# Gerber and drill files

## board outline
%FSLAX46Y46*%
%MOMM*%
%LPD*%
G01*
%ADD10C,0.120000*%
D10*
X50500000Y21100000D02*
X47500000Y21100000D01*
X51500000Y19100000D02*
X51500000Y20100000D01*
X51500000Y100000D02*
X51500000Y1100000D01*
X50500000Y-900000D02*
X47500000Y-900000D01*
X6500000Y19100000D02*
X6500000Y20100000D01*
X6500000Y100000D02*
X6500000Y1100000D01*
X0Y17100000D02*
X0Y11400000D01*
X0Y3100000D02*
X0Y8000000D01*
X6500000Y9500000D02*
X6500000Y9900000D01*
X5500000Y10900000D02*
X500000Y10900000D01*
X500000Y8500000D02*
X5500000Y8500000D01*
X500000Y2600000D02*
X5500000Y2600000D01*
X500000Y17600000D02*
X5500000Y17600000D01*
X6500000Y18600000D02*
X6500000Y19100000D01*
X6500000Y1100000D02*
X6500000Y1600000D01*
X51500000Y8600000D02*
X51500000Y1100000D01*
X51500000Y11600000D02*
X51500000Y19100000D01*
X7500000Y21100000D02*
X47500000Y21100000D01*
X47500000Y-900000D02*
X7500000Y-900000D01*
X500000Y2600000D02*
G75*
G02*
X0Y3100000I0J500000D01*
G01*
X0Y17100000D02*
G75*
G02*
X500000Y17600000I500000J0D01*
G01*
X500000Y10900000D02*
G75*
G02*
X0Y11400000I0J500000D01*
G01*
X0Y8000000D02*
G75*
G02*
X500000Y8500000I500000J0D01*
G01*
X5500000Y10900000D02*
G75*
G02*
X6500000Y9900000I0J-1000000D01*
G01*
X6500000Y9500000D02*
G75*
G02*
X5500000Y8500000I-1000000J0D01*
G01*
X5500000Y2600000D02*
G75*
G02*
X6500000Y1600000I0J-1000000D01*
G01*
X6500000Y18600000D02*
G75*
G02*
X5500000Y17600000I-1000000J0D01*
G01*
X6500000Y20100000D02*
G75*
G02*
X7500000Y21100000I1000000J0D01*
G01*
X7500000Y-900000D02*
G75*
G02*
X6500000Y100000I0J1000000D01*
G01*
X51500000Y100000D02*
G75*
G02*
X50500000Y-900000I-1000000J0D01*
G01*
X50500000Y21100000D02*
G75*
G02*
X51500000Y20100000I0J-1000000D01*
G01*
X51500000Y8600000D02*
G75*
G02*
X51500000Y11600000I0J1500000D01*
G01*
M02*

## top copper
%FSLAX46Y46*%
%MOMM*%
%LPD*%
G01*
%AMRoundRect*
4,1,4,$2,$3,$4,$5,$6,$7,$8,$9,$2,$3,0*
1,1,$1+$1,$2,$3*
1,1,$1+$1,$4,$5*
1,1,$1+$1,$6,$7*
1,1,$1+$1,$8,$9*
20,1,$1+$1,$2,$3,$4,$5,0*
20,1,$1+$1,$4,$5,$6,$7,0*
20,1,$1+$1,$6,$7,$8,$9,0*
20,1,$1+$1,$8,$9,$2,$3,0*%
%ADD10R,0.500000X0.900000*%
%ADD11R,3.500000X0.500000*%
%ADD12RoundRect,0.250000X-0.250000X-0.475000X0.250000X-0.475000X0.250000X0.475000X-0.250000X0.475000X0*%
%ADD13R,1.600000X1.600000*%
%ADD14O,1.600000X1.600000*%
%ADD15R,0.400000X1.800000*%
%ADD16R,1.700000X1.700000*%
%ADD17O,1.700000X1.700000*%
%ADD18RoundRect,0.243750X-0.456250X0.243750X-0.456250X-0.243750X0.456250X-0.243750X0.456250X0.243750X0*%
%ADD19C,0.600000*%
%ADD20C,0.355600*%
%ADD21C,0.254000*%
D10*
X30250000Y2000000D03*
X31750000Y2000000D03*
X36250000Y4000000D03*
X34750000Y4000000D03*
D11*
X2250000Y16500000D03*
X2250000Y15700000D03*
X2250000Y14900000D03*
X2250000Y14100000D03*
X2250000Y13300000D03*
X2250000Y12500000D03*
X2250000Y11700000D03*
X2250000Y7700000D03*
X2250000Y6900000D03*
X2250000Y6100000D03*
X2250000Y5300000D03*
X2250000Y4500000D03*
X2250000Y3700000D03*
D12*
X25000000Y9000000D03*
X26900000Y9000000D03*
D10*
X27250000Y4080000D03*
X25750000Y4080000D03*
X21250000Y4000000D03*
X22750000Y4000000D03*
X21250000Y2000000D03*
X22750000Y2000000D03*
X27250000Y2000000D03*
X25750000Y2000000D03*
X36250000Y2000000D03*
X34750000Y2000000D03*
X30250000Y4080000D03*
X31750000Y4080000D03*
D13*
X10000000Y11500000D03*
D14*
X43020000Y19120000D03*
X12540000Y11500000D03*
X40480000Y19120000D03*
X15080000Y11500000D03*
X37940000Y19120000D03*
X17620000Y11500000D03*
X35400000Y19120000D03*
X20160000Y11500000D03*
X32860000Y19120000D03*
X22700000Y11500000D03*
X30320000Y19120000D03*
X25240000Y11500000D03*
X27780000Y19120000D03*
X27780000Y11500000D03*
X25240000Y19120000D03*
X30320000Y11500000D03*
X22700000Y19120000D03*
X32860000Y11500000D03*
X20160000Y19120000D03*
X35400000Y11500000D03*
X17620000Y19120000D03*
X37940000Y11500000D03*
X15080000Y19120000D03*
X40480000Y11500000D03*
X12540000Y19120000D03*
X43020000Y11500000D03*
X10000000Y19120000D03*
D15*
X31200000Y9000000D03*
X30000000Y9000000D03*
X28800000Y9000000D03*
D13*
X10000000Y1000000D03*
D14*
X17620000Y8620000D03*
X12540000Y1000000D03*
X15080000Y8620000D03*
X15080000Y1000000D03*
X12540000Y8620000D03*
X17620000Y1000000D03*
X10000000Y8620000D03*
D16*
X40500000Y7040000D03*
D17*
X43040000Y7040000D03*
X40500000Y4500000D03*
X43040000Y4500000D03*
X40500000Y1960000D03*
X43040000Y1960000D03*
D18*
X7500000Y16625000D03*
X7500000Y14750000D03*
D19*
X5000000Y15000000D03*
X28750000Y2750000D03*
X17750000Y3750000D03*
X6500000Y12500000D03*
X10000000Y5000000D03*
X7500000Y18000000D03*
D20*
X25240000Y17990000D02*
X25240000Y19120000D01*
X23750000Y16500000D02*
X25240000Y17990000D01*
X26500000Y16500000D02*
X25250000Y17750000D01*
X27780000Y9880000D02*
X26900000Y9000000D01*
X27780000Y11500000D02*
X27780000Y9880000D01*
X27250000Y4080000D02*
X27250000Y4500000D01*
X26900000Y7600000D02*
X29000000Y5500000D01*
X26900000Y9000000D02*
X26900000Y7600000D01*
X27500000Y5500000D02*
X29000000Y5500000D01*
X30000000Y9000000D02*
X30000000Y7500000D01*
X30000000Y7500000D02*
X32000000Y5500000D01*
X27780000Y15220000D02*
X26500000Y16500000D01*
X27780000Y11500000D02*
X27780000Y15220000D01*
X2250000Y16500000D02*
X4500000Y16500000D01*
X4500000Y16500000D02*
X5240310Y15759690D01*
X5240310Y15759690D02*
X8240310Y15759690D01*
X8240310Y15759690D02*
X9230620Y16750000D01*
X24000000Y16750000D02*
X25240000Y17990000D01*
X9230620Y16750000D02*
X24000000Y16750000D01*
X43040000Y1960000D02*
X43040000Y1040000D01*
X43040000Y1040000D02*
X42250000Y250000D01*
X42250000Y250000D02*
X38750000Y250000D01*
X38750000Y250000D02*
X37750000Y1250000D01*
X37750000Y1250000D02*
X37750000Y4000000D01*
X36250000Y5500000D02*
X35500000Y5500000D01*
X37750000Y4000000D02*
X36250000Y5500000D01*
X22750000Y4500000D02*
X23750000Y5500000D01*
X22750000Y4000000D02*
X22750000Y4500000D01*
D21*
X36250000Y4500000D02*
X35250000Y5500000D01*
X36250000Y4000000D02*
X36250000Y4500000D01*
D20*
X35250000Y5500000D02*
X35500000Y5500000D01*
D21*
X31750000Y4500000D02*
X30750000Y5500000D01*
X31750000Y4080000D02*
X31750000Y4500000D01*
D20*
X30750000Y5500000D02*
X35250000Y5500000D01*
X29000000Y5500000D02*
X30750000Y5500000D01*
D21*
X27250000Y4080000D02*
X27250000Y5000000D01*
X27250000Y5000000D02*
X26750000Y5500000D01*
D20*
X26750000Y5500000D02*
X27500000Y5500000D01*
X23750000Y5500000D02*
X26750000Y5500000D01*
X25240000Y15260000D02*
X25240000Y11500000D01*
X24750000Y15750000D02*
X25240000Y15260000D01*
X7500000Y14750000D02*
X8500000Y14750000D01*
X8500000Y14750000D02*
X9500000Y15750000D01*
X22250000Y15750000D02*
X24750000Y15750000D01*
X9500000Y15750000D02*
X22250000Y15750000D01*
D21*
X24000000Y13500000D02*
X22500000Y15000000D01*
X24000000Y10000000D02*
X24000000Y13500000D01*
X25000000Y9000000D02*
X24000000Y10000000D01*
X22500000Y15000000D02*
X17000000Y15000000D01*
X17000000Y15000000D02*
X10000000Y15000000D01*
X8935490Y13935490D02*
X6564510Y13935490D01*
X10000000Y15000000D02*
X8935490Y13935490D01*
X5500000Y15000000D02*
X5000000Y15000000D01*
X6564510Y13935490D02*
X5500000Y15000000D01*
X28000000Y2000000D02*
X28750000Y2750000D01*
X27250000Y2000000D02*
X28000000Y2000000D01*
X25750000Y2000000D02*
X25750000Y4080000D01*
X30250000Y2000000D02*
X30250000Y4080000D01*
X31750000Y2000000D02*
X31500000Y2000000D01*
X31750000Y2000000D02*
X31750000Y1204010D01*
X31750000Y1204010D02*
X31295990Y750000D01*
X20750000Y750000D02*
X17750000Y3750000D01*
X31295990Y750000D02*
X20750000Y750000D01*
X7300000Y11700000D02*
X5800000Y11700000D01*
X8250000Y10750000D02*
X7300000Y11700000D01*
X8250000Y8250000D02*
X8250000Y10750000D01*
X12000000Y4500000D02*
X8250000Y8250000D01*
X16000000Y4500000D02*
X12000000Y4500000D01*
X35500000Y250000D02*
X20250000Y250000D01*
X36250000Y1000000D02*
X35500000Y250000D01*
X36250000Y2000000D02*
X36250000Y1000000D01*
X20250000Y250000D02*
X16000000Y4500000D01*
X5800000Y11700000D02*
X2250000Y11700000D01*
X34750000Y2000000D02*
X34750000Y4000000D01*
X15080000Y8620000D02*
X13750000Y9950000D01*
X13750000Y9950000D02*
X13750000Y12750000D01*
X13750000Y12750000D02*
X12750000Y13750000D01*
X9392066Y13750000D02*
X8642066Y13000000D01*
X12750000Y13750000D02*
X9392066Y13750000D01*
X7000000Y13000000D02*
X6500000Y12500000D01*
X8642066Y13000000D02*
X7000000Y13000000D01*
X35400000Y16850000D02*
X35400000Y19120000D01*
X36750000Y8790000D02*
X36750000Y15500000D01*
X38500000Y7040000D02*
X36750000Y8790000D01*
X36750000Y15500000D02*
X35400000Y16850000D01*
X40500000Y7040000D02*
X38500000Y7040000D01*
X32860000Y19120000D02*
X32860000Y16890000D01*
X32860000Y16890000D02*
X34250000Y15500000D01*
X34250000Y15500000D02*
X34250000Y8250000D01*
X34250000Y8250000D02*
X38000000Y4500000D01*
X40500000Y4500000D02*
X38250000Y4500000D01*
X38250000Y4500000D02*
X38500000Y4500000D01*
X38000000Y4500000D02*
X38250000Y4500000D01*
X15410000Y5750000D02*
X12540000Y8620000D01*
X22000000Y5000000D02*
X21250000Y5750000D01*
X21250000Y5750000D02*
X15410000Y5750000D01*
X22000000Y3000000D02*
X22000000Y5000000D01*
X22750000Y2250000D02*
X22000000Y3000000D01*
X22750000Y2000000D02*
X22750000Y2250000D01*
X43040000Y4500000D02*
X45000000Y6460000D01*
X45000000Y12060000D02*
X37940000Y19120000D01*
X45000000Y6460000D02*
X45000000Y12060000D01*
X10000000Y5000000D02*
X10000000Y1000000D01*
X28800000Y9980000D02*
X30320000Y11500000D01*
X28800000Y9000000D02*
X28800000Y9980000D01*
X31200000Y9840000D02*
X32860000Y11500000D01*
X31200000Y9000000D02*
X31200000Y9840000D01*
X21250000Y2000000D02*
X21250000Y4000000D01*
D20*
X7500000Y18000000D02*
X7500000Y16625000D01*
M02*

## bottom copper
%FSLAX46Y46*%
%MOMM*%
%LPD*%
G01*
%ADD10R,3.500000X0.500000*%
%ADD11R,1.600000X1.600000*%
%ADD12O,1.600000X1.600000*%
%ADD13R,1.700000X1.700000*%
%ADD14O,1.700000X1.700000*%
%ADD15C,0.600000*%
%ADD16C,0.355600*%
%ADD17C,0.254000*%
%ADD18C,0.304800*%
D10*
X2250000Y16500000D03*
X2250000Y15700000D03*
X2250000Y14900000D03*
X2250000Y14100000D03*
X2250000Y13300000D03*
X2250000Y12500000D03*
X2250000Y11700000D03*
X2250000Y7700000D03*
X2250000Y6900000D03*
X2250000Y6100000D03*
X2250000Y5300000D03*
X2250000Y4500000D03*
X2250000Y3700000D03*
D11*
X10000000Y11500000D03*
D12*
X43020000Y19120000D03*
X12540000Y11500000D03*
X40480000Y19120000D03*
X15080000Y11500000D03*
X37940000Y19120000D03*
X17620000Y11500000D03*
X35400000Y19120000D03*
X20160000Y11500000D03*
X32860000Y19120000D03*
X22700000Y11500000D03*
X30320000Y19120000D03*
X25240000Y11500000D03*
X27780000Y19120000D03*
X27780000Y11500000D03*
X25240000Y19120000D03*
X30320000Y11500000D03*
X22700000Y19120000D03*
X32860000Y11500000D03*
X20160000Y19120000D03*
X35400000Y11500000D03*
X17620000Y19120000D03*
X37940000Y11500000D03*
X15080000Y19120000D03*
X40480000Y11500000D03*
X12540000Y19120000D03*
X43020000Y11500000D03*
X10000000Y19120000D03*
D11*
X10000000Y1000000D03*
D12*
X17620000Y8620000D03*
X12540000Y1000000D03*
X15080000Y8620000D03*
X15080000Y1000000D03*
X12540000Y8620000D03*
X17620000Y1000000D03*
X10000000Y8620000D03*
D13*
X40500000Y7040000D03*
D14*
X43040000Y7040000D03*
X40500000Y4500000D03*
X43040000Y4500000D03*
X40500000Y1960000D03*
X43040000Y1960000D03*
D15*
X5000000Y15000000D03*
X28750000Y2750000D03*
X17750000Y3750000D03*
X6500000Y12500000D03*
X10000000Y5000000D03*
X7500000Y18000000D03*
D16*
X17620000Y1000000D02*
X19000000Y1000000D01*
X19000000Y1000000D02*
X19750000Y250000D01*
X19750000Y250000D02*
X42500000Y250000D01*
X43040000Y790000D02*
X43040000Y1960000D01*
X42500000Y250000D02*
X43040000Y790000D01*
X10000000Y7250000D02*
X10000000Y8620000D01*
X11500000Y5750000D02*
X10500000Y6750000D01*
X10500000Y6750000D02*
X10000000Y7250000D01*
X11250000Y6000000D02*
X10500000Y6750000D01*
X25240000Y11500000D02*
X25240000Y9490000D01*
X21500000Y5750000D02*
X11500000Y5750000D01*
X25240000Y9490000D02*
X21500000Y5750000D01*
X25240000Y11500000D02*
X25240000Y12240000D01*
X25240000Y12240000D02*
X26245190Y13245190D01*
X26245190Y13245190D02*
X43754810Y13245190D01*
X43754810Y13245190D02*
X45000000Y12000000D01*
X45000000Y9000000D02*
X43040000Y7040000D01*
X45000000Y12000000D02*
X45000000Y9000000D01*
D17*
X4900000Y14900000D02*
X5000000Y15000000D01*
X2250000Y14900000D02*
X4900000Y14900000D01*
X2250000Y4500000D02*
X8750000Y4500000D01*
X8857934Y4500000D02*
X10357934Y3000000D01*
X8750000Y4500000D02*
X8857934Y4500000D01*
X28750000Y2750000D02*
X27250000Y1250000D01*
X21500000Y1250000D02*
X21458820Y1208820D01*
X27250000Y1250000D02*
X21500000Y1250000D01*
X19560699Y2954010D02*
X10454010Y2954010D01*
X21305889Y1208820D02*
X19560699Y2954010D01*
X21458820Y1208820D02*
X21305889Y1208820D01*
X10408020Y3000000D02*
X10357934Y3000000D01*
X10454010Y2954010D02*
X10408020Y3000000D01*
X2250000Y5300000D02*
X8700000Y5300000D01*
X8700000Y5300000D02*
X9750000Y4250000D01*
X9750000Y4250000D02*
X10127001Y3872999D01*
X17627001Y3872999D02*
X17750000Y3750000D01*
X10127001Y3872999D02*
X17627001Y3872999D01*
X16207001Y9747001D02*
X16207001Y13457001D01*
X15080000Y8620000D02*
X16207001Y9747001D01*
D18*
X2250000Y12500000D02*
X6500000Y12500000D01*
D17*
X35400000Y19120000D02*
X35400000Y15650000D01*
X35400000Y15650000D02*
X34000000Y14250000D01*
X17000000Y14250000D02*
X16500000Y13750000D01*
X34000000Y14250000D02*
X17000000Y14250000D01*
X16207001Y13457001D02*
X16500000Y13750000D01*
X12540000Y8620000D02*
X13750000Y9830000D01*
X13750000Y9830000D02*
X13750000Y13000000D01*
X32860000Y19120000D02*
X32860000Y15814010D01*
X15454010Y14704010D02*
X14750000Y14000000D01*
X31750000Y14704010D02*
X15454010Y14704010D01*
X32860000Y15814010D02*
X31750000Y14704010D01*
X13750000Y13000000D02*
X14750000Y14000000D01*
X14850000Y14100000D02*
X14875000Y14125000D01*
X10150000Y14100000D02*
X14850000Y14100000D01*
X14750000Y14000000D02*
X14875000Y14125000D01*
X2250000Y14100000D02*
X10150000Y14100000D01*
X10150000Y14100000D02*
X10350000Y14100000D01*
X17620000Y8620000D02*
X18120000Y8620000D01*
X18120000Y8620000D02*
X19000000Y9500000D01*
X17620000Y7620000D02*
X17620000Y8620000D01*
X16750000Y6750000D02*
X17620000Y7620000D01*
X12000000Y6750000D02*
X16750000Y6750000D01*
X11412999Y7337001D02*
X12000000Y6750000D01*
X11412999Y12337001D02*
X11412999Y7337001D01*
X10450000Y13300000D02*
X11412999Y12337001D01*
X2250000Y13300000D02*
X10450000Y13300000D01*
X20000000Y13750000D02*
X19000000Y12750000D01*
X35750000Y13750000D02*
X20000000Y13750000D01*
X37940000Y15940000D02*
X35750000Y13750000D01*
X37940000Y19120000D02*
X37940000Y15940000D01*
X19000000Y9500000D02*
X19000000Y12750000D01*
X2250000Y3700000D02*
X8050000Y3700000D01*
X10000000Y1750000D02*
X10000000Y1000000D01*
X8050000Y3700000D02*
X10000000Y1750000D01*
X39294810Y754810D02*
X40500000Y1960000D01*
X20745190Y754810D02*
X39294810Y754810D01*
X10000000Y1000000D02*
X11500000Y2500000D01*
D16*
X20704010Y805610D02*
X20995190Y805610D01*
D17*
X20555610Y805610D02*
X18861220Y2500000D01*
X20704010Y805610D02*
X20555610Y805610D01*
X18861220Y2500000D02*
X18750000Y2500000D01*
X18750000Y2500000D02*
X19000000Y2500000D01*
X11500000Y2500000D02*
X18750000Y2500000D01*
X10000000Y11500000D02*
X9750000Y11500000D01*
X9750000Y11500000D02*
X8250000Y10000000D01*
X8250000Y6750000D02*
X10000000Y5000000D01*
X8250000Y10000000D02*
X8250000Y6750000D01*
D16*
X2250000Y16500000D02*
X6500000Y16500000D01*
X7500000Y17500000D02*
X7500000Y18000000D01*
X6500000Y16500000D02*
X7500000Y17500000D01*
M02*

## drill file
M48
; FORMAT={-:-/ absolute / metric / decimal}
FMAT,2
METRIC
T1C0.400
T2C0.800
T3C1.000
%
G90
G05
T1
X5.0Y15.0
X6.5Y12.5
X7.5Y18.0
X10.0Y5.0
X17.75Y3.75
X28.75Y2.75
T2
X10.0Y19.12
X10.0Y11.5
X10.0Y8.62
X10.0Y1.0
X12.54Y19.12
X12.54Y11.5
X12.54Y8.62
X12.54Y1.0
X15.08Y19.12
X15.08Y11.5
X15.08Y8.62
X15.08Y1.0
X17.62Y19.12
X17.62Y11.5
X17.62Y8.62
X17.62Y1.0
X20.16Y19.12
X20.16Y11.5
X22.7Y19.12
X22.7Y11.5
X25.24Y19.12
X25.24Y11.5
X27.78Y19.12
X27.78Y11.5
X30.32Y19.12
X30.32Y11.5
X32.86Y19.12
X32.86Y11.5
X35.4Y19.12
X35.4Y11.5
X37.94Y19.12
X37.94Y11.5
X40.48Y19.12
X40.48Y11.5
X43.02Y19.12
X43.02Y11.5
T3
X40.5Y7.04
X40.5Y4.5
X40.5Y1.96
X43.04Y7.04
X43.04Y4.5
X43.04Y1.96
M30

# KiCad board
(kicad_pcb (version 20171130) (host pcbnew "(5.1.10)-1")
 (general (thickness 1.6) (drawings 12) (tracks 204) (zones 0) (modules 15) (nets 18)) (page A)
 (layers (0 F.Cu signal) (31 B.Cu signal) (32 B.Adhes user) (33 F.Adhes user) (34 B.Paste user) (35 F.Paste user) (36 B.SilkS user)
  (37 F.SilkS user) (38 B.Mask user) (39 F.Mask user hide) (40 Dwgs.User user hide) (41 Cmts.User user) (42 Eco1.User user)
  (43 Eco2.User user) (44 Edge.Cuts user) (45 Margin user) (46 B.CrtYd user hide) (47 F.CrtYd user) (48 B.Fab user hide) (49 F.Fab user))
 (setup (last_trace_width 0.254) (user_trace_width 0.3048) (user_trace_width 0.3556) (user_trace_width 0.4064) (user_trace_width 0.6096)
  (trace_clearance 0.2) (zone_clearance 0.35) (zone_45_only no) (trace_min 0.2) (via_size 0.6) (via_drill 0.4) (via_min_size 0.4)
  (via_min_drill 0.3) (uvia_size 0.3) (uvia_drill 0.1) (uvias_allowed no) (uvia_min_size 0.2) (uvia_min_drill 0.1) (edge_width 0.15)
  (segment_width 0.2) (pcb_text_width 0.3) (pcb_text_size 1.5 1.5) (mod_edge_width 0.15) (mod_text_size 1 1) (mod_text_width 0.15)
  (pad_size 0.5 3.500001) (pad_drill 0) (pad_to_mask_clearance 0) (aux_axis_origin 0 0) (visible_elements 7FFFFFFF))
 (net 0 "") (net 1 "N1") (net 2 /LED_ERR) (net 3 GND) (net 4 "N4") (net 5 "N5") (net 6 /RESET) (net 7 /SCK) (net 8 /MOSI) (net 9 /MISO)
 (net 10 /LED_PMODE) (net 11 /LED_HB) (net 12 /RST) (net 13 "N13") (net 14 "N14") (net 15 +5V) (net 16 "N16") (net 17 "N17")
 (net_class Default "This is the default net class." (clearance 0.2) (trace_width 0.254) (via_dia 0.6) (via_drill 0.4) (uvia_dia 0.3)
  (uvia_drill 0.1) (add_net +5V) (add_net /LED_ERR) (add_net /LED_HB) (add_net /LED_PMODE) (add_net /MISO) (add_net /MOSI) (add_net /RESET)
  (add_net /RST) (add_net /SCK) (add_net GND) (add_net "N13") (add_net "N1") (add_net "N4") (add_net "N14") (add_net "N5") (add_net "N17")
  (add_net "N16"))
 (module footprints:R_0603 (layer F.Cu) (at 31 -2)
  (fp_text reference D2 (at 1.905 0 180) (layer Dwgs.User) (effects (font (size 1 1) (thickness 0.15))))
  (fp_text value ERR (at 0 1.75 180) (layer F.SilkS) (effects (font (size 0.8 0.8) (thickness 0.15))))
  (pad 1 smd rect (at -0.75 0) (size 0.5 0.9) (layers F.Cu F.Paste F.Mask) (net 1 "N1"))
  (pad 2 smd rect (at 0.75 0) (size 0.5 0.9) (layers F.Cu F.Paste F.Mask) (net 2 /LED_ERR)))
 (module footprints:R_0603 (layer F.Cu) (at 35.5 -4 180)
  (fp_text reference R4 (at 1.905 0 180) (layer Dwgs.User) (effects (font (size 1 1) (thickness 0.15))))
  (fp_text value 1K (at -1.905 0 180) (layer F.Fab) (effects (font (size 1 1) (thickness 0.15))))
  (pad 1 smd rect (at -0.75 0 180) (size 0.5 0.9) (layers F.Cu F.Paste F.Mask) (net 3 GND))
  (pad 2 smd rect (at 0.75 0 180) (size 0.5 0.9) (layers F.Cu F.Paste F.Mask) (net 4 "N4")))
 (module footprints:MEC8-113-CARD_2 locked (layer F.Cu) (at 0 -0.1 90)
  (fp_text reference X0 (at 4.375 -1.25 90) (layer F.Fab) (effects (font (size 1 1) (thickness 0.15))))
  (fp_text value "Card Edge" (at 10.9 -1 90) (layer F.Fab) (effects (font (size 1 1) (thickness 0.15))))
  (fp_line (start 21 50.5) (end 21 47.5) (layer Edge.Cuts) (width 0.12))
  (fp_line (start 19 51.5) (end 20 51.5) (layer Edge.Cuts) (width 0.12))
  (fp_line (start 0 51.5) (end 1 51.5) (layer Edge.Cuts) (width 0.12))
  (fp_line (start -1 50.5) (end -1 47.5) (layer Edge.Cuts) (width 0.12))
  (fp_line (start 19 6.5) (end 20 6.5) (layer Edge.Cuts) (width 0.12))
  (fp_line (start 0 6.5) (end 1 6.5) (layer Edge.Cuts) (width 0.12))
  (fp_line (start 17 0) (end 11.3 0) (layer Edge.Cuts) (width 0.12))
  (fp_line (start 3 0) (end 7.9 0) (layer Edge.Cuts) (width 0.12))
  (fp_line (start 9.4 6.5) (end 9.8 6.5) (layer Edge.Cuts) (width 0.12))
  (fp_line (start 10.8 5.5) (end 10.8 0.5) (layer Edge.Cuts) (width 0.12))
  (fp_line (start 8.4 0.5) (end 8.4 5.5) (layer Edge.Cuts) (width 0.12))
  (fp_line (start 2.5 0.5) (end 2.5 5.5) (layer Edge.Cuts) (width 0.12))
  (fp_line (start 17.5 0.5) (end 17.5 5.5) (layer Edge.Cuts) (width 0.12))
  (fp_line (start 18.5 6.5) (end 19 6.5) (layer Edge.Cuts) (width 0.12))
  (fp_line (start 1 6.5) (end 1.5 6.5) (layer Edge.Cuts) (width 0.12))
  (fp_line (start 8.5 51.5) (end 1 51.5) (layer Edge.Cuts) (width 0.12))
  (fp_line (start 11.5 51.5) (end 19 51.5) (layer Edge.Cuts) (width 0.12))
  (fp_line (start 21 7.5) (end 21 47.5) (layer Edge.Cuts) (width 0.12))
  (fp_line (start -1 47.5) (end -1 7.5) (layer Edge.Cuts) (width 0.12))
  (fp_arc (start 3 0.5) (end 3 0) (angle -90) (layer Edge.Cuts) (width 0.12))
  (fp_arc (start 17 0.5) (end 17.5 0.5) (angle -90) (layer Edge.Cuts) (width 0.12))
  (fp_arc (start 11.3 0.5) (end 11.3 0) (angle -90) (layer Edge.Cuts) (width 0.12))
  (fp_arc (start 7.9 0.5) (end 8.4 0.5) (angle -90) (layer Edge.Cuts) (width 0.12))
  (fp_arc (start 9.8 5.5) (end 9.8 6.5) (angle -90) (layer Edge.Cuts) (width 0.12))
  (fp_arc (start 9.4 5.5) (end 8.4 5.5) (angle -90) (layer Edge.Cuts) (width 0.12))
  (fp_arc (start 1.5 5.5) (end 1.5 6.5) (angle -90) (layer Edge.Cuts) (width 0.12))
  (fp_arc (start 18.5 5.5) (end 17.5 5.5) (angle -90) (layer Edge.Cuts) (width 0.12))
  (fp_arc (start 20 7.5) (end 21 7.5) (angle -90) (layer Edge.Cuts) (width 0.12))
  (fp_arc (start 0 7.5) (end 0 6.5) (angle -90) (layer Edge.Cuts) (width 0.12))
  (fp_arc (start 0 50.5) (end -1 50.5) (angle -90) (layer Edge.Cuts) (width 0.12))
  (fp_arc (start 20 50.5) (end 20 51.5) (angle -90) (layer Edge.Cuts) (width 0.12))
  (fp_arc (start 10 51.5) (end 11.5 51.5) (angle -180) (layer Edge.Cuts) (width 0.12))
  (pad 13 smd rect (at 16.4 2.25 90) (size 0.5 3.5) (layers B.Cu B.Paste B.Mask) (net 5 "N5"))
  (pad 26 smd rect (at 16.4 2.25 90) (size 0.5 3.5) (layers F.Cu F.Paste F.Mask) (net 3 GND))
  (pad 12 smd rect (at 15.6 2.25 90) (size 0.5 3.5) (layers B.Cu B.Paste B.Mask))
  (pad 25 smd rect (at 15.6 2.25 90) (size 0.5 3.5) (layers F.Cu F.Paste F.Mask))
  (pad 11 smd rect (at 14.8 2.25 90) (size 0.5 3.5) (layers B.Cu B.Paste B.Mask) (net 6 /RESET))
  (pad 24 smd rect (at 14.8 2.25 90) (size 0.5 3.5) (layers F.Cu F.Paste F.Mask))
  (pad 10 smd rect (at 14 2.25 90) (size 0.5 3.5) (layers B.Cu B.Paste B.Mask) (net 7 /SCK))
  (pad 23 smd rect (at 14 2.25 90) (size 0.5 3.5) (layers F.Cu F.Paste F.Mask))
  (pad 9 smd rect (at 13.2 2.25 90) (size 0.5 3.5) (layers B.Cu B.Paste B.Mask) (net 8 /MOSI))
  (pad 22 smd rect (at 13.2 2.25 90) (size 0.5 3.5) (layers F.Cu F.Paste F.Mask))
  (pad 8 smd rect (at 12.4 2.25 90) (size 0.5 3.5) (layers B.Cu B.Paste B.Mask) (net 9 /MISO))
  (pad 21 smd rect (at 12.4 2.25 90) (size 0.5 3.5) (layers F.Cu F.Paste F.Mask))
  (pad 7 smd rect (at 11.6 2.25 90) (size 0.5 3.5) (layers B.Cu B.Paste B.Mask))
  (pad 20 smd rect (at 11.6 2.25 90) (size 0.5 3.5) (layers F.Cu F.Paste F.Mask) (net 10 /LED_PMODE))
  (pad 6 smd rect (at 7.6 2.25 90) (size 0.5 3.5) (layers B.Cu B.Paste B.Mask))
  (pad 19 smd rect (at 7.6 2.25 90) (size 0.5 3.5) (layers F.Cu F.Paste F.Mask))
  (pad 5 smd rect (at 6.8 2.25 90) (size 0.5 3.5) (layers B.Cu B.Paste B.Mask))
  (pad 18 smd rect (at 6.8 2.25 90) (size 0.5 3.5) (layers F.Cu F.Paste F.Mask))
  (pad 4 smd rect (at 6 2.25 90) (size 0.5 3.5) (layers B.Cu B.Paste B.Mask))
  (pad 17 smd rect (at 6 2.25 90) (size 0.5 3.5) (layers F.Cu F.Paste F.Mask))
  (pad 3 smd rect (at 5.2 2.25 90) (size 0.5 3.5) (layers B.Cu B.Paste B.Mask) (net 2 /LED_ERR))
  (pad 16 smd rect (at 5.2 2.25 90) (size 0.5 3.5) (layers F.Cu F.Paste F.Mask))
  (pad 2 smd rect (at 4.4 2.25 90) (size 0.5 3.5) (layers B.Cu B.Paste B.Mask) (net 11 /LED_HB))
  (pad 15 smd rect (at 4.4 2.25 90) (size 0.5 3.5) (layers F.Cu F.Paste F.Mask))
  (pad 1 smd rect (at 3.6 2.25 90) (size 0.5 3.5) (layers B.Cu B.Paste B.Mask) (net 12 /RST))
  (pad 14 smd rect (at 3.6 2.25 90) (size 0.5 3.5) (layers F.Cu F.Paste F.Mask)))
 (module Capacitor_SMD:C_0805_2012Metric (layer F.Cu) (at 25.95 -9)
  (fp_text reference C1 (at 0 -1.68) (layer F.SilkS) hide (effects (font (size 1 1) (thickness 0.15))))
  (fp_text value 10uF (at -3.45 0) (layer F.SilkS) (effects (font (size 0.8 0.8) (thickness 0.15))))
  (pad 1 smd roundrect (at -0.95 0) (size 1 1.45) (layers F.Cu F.Paste F.Mask) (roundrect_rratio 0.25) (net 6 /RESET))
  (pad 2 smd roundrect (at 0.95 0) (size 1 1.45) (layers F.Cu F.Paste F.Mask) (roundrect_rratio 0.25) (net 3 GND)))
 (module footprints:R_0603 (layer F.Cu) (at 26.5 -4.08 180)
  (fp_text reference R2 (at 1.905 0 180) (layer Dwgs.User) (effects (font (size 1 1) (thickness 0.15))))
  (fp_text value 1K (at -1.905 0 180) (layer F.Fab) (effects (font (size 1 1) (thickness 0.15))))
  (pad 1 smd rect (at -0.75 0 180) (size 0.5 0.9) (layers F.Cu F.Paste F.Mask) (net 3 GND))
  (pad 2 smd rect (at 0.75 0 180) (size 0.5 0.9) (layers F.Cu F.Paste F.Mask) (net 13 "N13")))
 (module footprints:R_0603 (layer F.Cu) (at 22 -4 180)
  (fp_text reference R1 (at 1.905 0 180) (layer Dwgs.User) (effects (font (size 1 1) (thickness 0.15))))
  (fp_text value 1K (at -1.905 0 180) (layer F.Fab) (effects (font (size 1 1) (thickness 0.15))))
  (pad 2 smd rect (at 0.75 0 180) (size 0.5 0.9) (layers F.Cu F.Paste F.Mask) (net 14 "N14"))
  (pad 1 smd rect (at -0.75 0 180) (size 0.5 0.9) (layers F.Cu F.Paste F.Mask) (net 3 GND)))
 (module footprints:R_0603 (layer F.Cu) (at 22 -2)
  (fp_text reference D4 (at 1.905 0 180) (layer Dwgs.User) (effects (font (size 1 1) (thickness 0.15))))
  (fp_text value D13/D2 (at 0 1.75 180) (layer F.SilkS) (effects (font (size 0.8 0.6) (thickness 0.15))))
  (pad 1 smd rect (at -0.75 0) (size 0.5 0.9) (layers F.Cu F.Paste F.Mask) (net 14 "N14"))
  (pad 2 smd rect (at 0.75 0) (size 0.5 0.9) (layers F.Cu F.Paste F.Mask) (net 7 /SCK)))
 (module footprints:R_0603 (layer F.Cu) (at 26.5 -2)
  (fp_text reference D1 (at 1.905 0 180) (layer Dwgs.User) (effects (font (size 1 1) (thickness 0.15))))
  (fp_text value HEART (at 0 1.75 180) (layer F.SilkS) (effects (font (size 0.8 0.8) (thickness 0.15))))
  (pad 2 smd rect (at 0.75 0) (size 0.5 0.9) (layers F.Cu F.Paste F.Mask) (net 11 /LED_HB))
  (pad 1 smd rect (at -0.75 0) (size 0.5 0.9) (layers F.Cu F.Paste F.Mask) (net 13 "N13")))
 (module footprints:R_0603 (layer F.Cu) (at 35.5 -2)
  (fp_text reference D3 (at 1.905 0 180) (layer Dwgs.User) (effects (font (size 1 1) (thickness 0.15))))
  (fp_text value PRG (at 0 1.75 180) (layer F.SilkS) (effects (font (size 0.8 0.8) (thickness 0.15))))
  (pad 2 smd rect (at 0.75 0) (size 0.5 0.9) (layers F.Cu F.Paste F.Mask) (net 10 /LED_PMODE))
  (pad 1 smd rect (at -0.75 0) (size 0.5 0.9) (layers F.Cu F.Paste F.Mask) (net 4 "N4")))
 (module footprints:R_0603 (layer F.Cu) (at 31 -4.08 180)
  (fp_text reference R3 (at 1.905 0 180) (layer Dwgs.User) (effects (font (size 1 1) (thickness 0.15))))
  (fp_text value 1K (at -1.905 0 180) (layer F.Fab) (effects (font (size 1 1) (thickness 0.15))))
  (pad 2 smd rect (at 0.75 0 180) (size 0.5 0.9) (layers F.Cu F.Paste F.Mask) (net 1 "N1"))
  (pad 1 smd rect (at -0.75 0 180) (size 0.5 0.9) (layers F.Cu F.Paste F.Mask) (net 3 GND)))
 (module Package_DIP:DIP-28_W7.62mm (layer F.Cu) (at 10 -11.5 90)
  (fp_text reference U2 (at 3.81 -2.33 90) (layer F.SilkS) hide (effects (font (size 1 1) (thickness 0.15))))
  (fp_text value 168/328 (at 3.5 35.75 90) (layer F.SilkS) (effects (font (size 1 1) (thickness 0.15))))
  (pad 1 thru_hole rect (at 0 0 90) (size 1.6 1.6) (drill 0.8) (layers *.Cu *.Mask) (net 12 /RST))
  (pad 15 thru_hole oval (at 7.62 33.02 90) (size 1.6 1.6) (drill 0.8) (layers *.Cu *.Mask))
  (pad 2 thru_hole oval (at 0 2.54 90) (size 1.6 1.6) (drill 0.8) (layers *.Cu *.Mask))
  (pad 16 thru_hole oval (at 7.62 30.48 90) (size 1.6 1.6) (drill 0.8) (layers *.Cu *.Mask))
  (pad 3 thru_hole oval (at 0 5.08 90) (size 1.6 1.6) (drill 0.8) (layers *.Cu *.Mask))
  (pad 17 thru_hole oval (at 7.62 27.94 90) (size 1.6 1.6) (drill 0.8) (layers *.Cu *.Mask) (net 8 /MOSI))
  (pad 4 thru_hole oval (at 0 7.62 90) (size 1.6 1.6) (drill 0.8) (layers *.Cu *.Mask))
  (pad 18 thru_hole oval (at 7.62 25.4 90) (size 1.6 1.6) (drill 0.8) (layers *.Cu *.Mask) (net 9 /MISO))
  (pad 5 thru_hole oval (at 0 10.16 90) (size 1.6 1.6) (drill 0.8) (layers *.Cu *.Mask))
  (pad 19 thru_hole oval (at 7.62 22.86 90) (size 1.6 1.6) (drill 0.8) (layers *.Cu *.Mask) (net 7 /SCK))
  (pad 6 thru_hole oval (at 0 12.7 90) (size 1.6 1.6) (drill 0.8) (layers *.Cu *.Mask))
  (pad 20 thru_hole oval (at 7.62 20.32 90) (size 1.6 1.6) (drill 0.8) (layers *.Cu *.Mask))
  (pad 7 thru_hole oval (at 0 15.24 90) (size 1.6 1.6) (drill 0.8) (layers *.Cu *.Mask) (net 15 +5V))
  (pad 21 thru_hole oval (at 7.62 17.78 90) (size 1.6 1.6) (drill 0.8) (layers *.Cu *.Mask))
  (pad 8 thru_hole oval (at 0 17.78 90) (size 1.6 1.6) (drill 0.8) (layers *.Cu *.Mask) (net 3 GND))
  (pad 22 thru_hole oval (at 7.62 15.24 90) (size 1.6 1.6) (drill 0.8) (layers *.Cu *.Mask) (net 3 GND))
  (pad 9 thru_hole oval (at 0 20.32 90) (size 1.6 1.6) (drill 0.8) (layers *.Cu *.Mask) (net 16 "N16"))
  (pad 23 thru_hole oval (at 7.62 12.7 90) (size 1.6 1.6) (drill 0.8) (layers *.Cu *.Mask))
  (pad 10 thru_hole oval (at 0 22.86 90) (size 1.6 1.6) (drill 0.8) (layers *.Cu *.Mask) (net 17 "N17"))
  (pad 24 thru_hole oval (at 7.62 10.16 90) (size 1.6 1.6) (drill 0.8) (layers *.Cu *.Mask))
  (pad 11 thru_hole oval (at 0 25.4 90) (size 1.6 1.6) (drill 0.8) (layers *.Cu *.Mask))
  (pad 25 thru_hole oval (at 7.62 7.62 90) (size 1.6 1.6) (drill 0.8) (layers *.Cu *.Mask))
  (pad 12 thru_hole oval (at 0 27.94 90) (size 1.6 1.6) (drill 0.8) (layers *.Cu *.Mask))
  (pad 26 thru_hole oval (at 7.62 5.08 90) (size 1.6 1.6) (drill 0.8) (layers *.Cu *.Mask))
  (pad 13 thru_hole oval (at 0 30.48 90) (size 1.6 1.6) (drill 0.8) (layers *.Cu *.Mask))
  (pad 27 thru_hole oval (at 7.62 2.54 90) (size 1.6 1.6) (drill 0.8) (layers *.Cu *.Mask))
  (pad 14 thru_hole oval (at 0 33.02 90) (size 1.6 1.6) (drill 0.8) (layers *.Cu *.Mask))
  (pad 28 thru_hole oval (at 7.62 0 90) (size 1.6 1.6) (drill 0.8) (layers *.Cu *.Mask)))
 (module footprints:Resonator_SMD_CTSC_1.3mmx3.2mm (layer F.Cu) (at 30 -9 180)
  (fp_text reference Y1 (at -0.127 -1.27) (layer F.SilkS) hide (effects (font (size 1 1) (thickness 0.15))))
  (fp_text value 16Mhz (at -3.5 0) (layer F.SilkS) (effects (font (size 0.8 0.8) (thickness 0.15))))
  (pad 1 smd rect (at -1.2 0 180) (size 0.4 1.8) (layers F.Cu F.Paste F.Mask) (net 17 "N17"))
  (pad 2 smd rect (at 0 0 180) (size 0.4 1.8) (layers F.Cu F.Paste F.Mask) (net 3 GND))
  (pad 3 smd rect (at 1.2 0 180) (size 0.4 1.8) (layers F.Cu F.Paste F.Mask) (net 16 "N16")))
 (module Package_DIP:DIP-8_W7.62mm (layer F.Cu) (at 10 -1 90)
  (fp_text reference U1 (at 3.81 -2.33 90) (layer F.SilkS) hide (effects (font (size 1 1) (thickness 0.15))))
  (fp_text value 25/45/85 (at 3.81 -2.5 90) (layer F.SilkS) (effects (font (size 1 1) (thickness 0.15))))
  (pad 1 thru_hole rect (at 0 0 90) (size 1.6 1.6) (drill 0.8) (layers *.Cu *.Mask) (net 12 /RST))
  (pad 5 thru_hole oval (at 7.62 7.62 90) (size 1.6 1.6) (drill 0.8) (layers *.Cu *.Mask) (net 8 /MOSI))
  (pad 2 thru_hole oval (at 0 2.54 90) (size 1.6 1.6) (drill 0.8) (layers *.Cu *.Mask))
  (pad 6 thru_hole oval (at 7.62 5.08 90) (size 1.6 1.6) (drill 0.8) (layers *.Cu *.Mask) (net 9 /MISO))
  (pad 3 thru_hole oval (at 0 5.08 90) (size 1.6 1.6) (drill 0.8) (layers *.Cu *.Mask))
  (pad 7 thru_hole oval (at 7.62 2.54 90) (size 1.6 1.6) (drill 0.8) (layers *.Cu *.Mask) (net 7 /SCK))
  (pad 4 thru_hole oval (at 0 7.62 90) (size 1.6 1.6) (drill 0.8) (layers *.Cu *.Mask) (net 3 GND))
  (pad 8 thru_hole oval (at 7.62 0 90) (size 1.6 1.6) (drill 0.8) (layers *.Cu *.Mask) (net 15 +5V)))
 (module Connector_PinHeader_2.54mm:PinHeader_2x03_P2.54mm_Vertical (layer F.Cu) (at 40.5 -7.04)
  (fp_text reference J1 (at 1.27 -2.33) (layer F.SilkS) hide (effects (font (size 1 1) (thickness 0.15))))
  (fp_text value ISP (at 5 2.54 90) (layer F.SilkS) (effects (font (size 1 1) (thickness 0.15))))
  (pad 1 thru_hole rect (at 0 0) (size 1.7 1.7) (drill 1) (layers *.Cu *.Mask) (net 9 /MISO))
  (pad 2 thru_hole oval (at 2.54 0) (size 1.7 1.7) (drill 1) (layers *.Cu *.Mask) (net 15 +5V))
  (pad 3 thru_hole oval (at 0 2.54) (size 1.7 1.7) (drill 1) (layers *.Cu *.Mask) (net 7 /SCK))
  (pad 4 thru_hole oval (at 2.54 2.54) (size 1.7 1.7) (drill 1) (layers *.Cu *.Mask) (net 8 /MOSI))
  (pad 5 thru_hole oval (at 0 5.08) (size 1.7 1.7) (drill 1) (layers *.Cu *.Mask) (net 12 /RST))
  (pad 6 thru_hole oval (at 2.54 5.08) (size 1.7 1.7) (drill 1) (layers *.Cu *.Mask) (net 3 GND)))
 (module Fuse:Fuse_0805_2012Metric (layer F.Cu) (at 7.5 -15.6875 270)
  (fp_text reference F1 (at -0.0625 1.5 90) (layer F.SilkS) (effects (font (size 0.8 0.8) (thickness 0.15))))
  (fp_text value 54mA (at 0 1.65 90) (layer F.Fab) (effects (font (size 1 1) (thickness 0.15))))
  (pad 1 smd roundrect (at -0.9375 0 270) (size 0.975 1.4) (layers F.Cu F.Paste F.Mask) (roundrect_rratio 0.25) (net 5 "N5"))
  (pad 2 smd roundrect (at 0.9375 0 270) (size 0.975 1.4) (layers F.Cu F.Paste F.Mask) (roundrect_rratio 0.25) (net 15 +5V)))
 (segment (start 25.24 -17.99) (end 25.24 -19.12) (width 0.3556) (layer F.Cu) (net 3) (status 20))
 (segment (start 23.75 -16.5) (end 25.24 -17.99) (width 0.3556) (layer F.Cu) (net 3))
 (segment (start 26.5 -16.5) (end 25.25 -17.75) (width 0.3556) (layer F.Cu) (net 3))
 (segment (start 27.78 -9.88) (end 26.9 -9) (width 0.3556) (layer F.Cu) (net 3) (status 20))
 (segment (start 27.78 -11.5) (end 27.78 -9.88) (width 0.3556) (layer F.Cu) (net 3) (status 10))
 (segment (start 27.25 -4.08) (end 27.25 -4.5) (width 0.3556) (layer F.Cu) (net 3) (status 30))
 (segment (start 26.9 -7.6) (end 29 -5.5) (width 0.3556) (layer F.Cu) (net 3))
 (segment (start 26.9 -9) (end 26.9 -7.6) (width 0.3556) (layer F.Cu) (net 3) (status 10))
 (segment (start 27.5 -5.5) (end 29 -5.5) (width 0.3556) (layer F.Cu) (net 3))
 (segment (start 30 -9) (end 30 -7.5) (width 0.3556) (layer F.Cu) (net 3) (status 10))
 (segment (start 30 -7.5) (end 32 -5.5) (width 0.3556) (layer F.Cu) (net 3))
 (segment (start 27.78 -15.22) (end 26.5 -16.5) (width 0.3556) (layer F.Cu) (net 3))
 (segment (start 27.78 -11.5) (end 27.78 -15.22) (width 0.3556) (layer F.Cu) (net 3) (status 10))
 (segment (start 2.25 -16.5) (end 4.5 -16.5) (width 0.3556) (layer F.Cu) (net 3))
 (segment (start 4.5 -16.5) (end 5.24031 -15.75969) (width 0.3556) (layer F.Cu) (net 3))
 (segment (start 5.24031 -15.75969) (end 8.24031 -15.75969) (width 0.3556) (layer F.Cu) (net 3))
 (segment (start 8.24031 -15.75969) (end 9.23062 -16.75) (width 0.3556) (layer F.Cu) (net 3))
 (segment (start 24 -16.75) (end 25.24 -17.99) (width 0.3556) (layer F.Cu) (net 3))
 (segment (start 9.23062 -16.75) (end 24 -16.75) (width 0.3556) (layer F.Cu) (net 3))
 (segment (start 17.62 -1) (end 19 -1) (width 0.3556) (layer B.Cu) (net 3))
 (segment (start 19 -1) (end 19.75 -0.25) (width 0.3556) (layer B.Cu) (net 3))
 (segment (start 19.75 -0.25) (end 42.5 -0.25) (width 0.3556) (layer B.Cu) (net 3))
 (segment (start 43.04 -0.79) (end 43.04 -1.96) (width 0.3556) (layer B.Cu) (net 3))
 (segment (start 42.5 -0.25) (end 43.04 -0.79) (width 0.3556) (layer B.Cu) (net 3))
 (segment (start 43.04 -1.96) (end 43.04 -1.04) (width 0.3556) (layer F.Cu) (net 3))
 (segment (start 43.04 -1.04) (end 42.25 -0.25) (width 0.3556) (layer F.Cu) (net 3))
 (segment (start 42.25 -0.25) (end 38.75 -0.25) (width 0.3556) (layer F.Cu) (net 3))
 (segment (start 38.75 -0.25) (end 37.75 -1.25) (width 0.3556) (layer F.Cu) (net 3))
 (segment (start 37.75 -1.25) (end 37.75 -4) (width 0.3556) (layer F.Cu) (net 3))
 (segment (start 36.25 -5.5) (end 35.5 -5.5) (width 0.3556) (layer F.Cu) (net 3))
 (segment (start 37.75 -4) (end 36.25 -5.5) (width 0.3556) (layer F.Cu) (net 3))
 (segment (start 22.75 -4.5) (end 23.75 -5.5) (width 0.3556) (layer F.Cu) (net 3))
 (segment (start 22.75 -4) (end 22.75 -4.5) (width 0.3556) (layer F.Cu) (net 3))
 (segment (start 36.25 -4.5) (end 35.25 -5.5) (width 0.254) (layer F.Cu) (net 3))
 (segment (start 36.25 -4) (end 36.25 -4.5) (width 0.254) (layer F.Cu) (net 3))
 (segment (start 35.25 -5.5) (end 35.5 -5.5) (width 0.3556) (layer F.Cu) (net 3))
 (segment (start 31.75 -4.5) (end 30.75 -5.5) (width 0.254) (layer F.Cu) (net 3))
 (segment (start 31.75 -4.08) (end 31.75 -4.5) (width 0.254) (layer F.Cu) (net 3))
 (segment (start 30.75 -5.5) (end 35.25 -5.5) (width 0.3556) (layer F.Cu) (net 3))
 (segment (start 29 -5.5) (end 30.75 -5.5) (width 0.3556) (layer F.Cu) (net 3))
 (segment (start 27.25 -4.08) (end 27.25 -5) (width 0.254) (layer F.Cu) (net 3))
 (segment (start 27.25 -5) (end 26.75 -5.5) (width 0.254) (layer F.Cu) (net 3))
 (segment (start 26.75 -5.5) (end 27.5 -5.5) (width 0.3556) (layer F.Cu) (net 3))
 (segment (start 23.75 -5.5) (end 26.75 -5.5) (width 0.3556) (layer F.Cu) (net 3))
 (segment (start 10 -7.25) (end 10 -8.62) (width 0.3556) (layer B.Cu) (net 15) (status 20))
 (segment (start 25.24 -15.26) (end 25.24 -11.5) (width 0.3556) (layer F.Cu) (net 15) (status 20))
 (segment (start 24.75 -15.75) (end 25.24 -15.26) (width 0.3556) (layer F.Cu) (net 15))
 (segment (start 11.5 -5.75) (end 10.5 -6.75) (width 0.3556) (layer B.Cu) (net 15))
 (segment (start 10.5 -6.75) (end 10 -7.25) (width 0.3556) (layer B.Cu) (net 15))
 (segment (start 11.25 -6) (end 10.5 -6.75) (width 0.3556) (layer B.Cu) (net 15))
 (segment (start 25.24 -11.5) (end 25.24 -9.49) (width 0.3556) (layer B.Cu) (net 15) (status 10))
 (segment (start 21.5 -5.75) (end 11.5 -5.75) (width 0.3556) (layer B.Cu) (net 15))
 (segment (start 25.24 -9.49) (end 21.5 -5.75) (width 0.3556) (layer B.Cu) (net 15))
 (segment (start 7.5 -14.75) (end 8.5 -14.75) (width 0.3556) (layer F.Cu) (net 15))
 (segment (start 8.5 -14.75) (end 9.5 -15.75) (width 0.3556) (layer F.Cu) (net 15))
 (segment (start 22.25 -15.75) (end 24.75 -15.75) (width 0.3556) (layer F.Cu) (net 15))
 (segment (start 9.5 -15.75) (end 22.25 -15.75) (width 0.3556) (layer F.Cu) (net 15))
 (segment (start 25.24 -11.5) (end 25.24 -12.24) (width 0.3556) (layer B.Cu) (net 15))
 (segment (start 25.24 -12.24) (end 26.24519 -13.24519) (width 0.3556) (layer B.Cu) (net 15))
 (segment (start 26.24519 -13.24519) (end 43.75481 -13.24519) (width 0.3556) (layer B.Cu) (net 15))
 (segment (start 43.75481 -13.24519) (end 45 -12) (width 0.3556) (layer B.Cu) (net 15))
 (segment (start 45 -9) (end 43.04 -7.04) (width 0.3556) (layer B.Cu) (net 15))
 (segment (start 45 -12) (end 45 -9) (width 0.3556) (layer B.Cu) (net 15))
 (segment (start 24 -13.5) (end 22.5 -15) (width 0.254) (layer F.Cu) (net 6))
 (segment (start 24 -10) (end 24 -13.5) (width 0.254) (layer F.Cu) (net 6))
 (segment (start 25 -9) (end 24 -10) (width 0.254) (layer F.Cu) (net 6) (status 10))
 (segment (start 22.5 -15) (end 17 -15) (width 0.254) (layer F.Cu) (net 6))
 (segment (start 17 -15) (end 10 -15) (width 0.254) (layer F.Cu) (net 6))
 (segment (start 8.93549 -13.93549) (end 6.56451 -13.93549) (width 0.254) (layer F.Cu) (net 6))
 (segment (start 10 -15) (end 8.93549 -13.93549) (width 0.254) (layer F.Cu) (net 6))
 (via (at 5 -15) (size 0.6) (drill 0.4) (layers F.Cu B.Cu) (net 6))
 (segment (start 5.5 -15) (end 5 -15) (width 0.254) (layer F.Cu) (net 6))
 (segment (start 6.56451 -13.93549) (end 5.5 -15) (width 0.254) (layer F.Cu) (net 6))
 (segment (start 4.9 -14.9) (end 5 -15) (width 0.254) (layer B.Cu) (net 6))
 (segment (start 2.25 -14.9) (end 4.9 -14.9) (width 0.254) (layer B.Cu) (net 6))
 (segment (start 2.25 -4.5) (end 8.75 -4.5) (width 0.254) (layer B.Cu) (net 11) (status 10))
 (segment (start 8.857934 -4.5) (end 10.357934 -3) (width 0.254) (layer B.Cu) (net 11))
 (segment (start 8.75 -4.5) (end 8.857934 -4.5) (width 0.254) (layer B.Cu) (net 11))
 (via (at 28.75 -2.75) (size 0.6) (drill 0.4) (layers F.Cu B.Cu) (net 11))
 (segment (start 28 -2) (end 28.75 -2.75) (width 0.254) (layer F.Cu) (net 11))
 (segment (start 27.25 -2) (end 28 -2) (width 0.254) (layer F.Cu) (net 11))
 (segment (start 28.75 -2.75) (end 27.25 -1.25) (width 0.254) (layer B.Cu) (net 11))
 (segment (start 21.5 -1.25) (end 21.45882 -1.20882) (width 0.254) (layer B.Cu) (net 11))
 (segment (start 27.25 -1.25) (end 21.5 -1.25) (width 0.254) (layer B.Cu) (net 11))
 (segment (start 19.560699 -2.95401) (end 10.45401 -2.95401) (width 0.254) (layer B.Cu) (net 11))
 (segment (start 21.305889 -1.20882) (end 19.560699 -2.95401) (width 0.254) (layer B.Cu) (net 11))
 (segment (start 21.45882 -1.20882) (end 21.305889 -1.20882) (width 0.254) (layer B.Cu) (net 11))
 (segment (start 10.40802 -3) (end 10.357934 -3) (width 0.254) (layer B.Cu) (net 11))
 (segment (start 10.45401 -2.95401) (end 10.40802 -3) (width 0.254) (layer B.Cu) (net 11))
 (segment (start 25.75 -2) (end 25.75 -4.08) (width 0.254) (layer F.Cu) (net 13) (status 30))
 (segment (start 30.25 -2) (end 30.25 -4.08) (width 0.254) (layer F.Cu) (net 1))
 (segment (start 2.25 -5.3) (end 8.7 -5.3) (width 0.254) (layer B.Cu) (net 2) (status 10))
 (segment (start 8.7 -5.3) (end 9.75 -4.25) (width 0.254) (layer B.Cu) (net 2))
 (segment (start 9.75 -4.25) (end 10.127001 -3.872999) (width 0.254) (layer B.Cu) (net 2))
 (segment (start 31.75 -2) (end 31.5 -2) (width 0.254) (layer F.Cu) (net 2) (status 30))
 (via (at 17.75 -3.75) (size 0.6) (drill 0.4) (layers F.Cu B.Cu) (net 2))
 (segment (start 17.627001 -3.872999) (end 17.75 -3.75) (width 0.254) (layer B.Cu) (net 2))
 (segment (start 10.127001 -3.872999) (end 17.627001 -3.872999) (width 0.254) (layer B.Cu) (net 2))
 (segment (start 31.75 -2) (end 31.75 -1.20401) (width 0.254) (layer F.Cu) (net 2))
 (segment (start 31.75 -1.20401) (end 31.29599 -0.75) (width 0.254) (layer F.Cu) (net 2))
 (segment (start 20.75 -0.75) (end 17.75 -3.75) (width 0.254) (layer F.Cu) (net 2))
 (segment (start 31.29599 -0.75) (end 20.75 -0.75) (width 0.254) (layer F.Cu) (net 2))
 (segment (start 7.3 -11.7) (end 5.8 -11.7) (width 0.254) (layer F.Cu) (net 10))
 (segment (start 8.25 -10.75) (end 7.3 -11.7) (width 0.254) (layer F.Cu) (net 10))
 (segment (start 8.25 -8.25) (end 8.25 -10.75) (width 0.254) (layer F.Cu) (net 10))
 (segment (start 12 -4.5) (end 8.25 -8.25) (width 0.254) (layer F.Cu) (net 10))
 (segment (start 16 -4.5) (end 12 -4.5) (width 0.254) (layer F.Cu) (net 10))
 (segment (start 35.5 -0.25) (end 20.25 -0.25) (width 0.254) (layer F.Cu) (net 10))
 (segment (start 36.25 -1) (end 35.5 -0.25) (width 0.254) (layer F.Cu) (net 10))
 (segment (start 36.25 -2) (end 36.25 -1) (width 0.254) (layer F.Cu) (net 10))
 (segment (start 20.25 -0.25) (end 16 -4.5) (width 0.254) (layer F.Cu) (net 10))
 (segment (start 5.8 -11.7) (end 2.25 -11.7) (width 0.254) (layer F.Cu) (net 10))
 (segment (start 34.75 -2) (end 34.75 -4) (width 0.254) (layer F.Cu) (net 4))
 (segment (start 16.207001 -9.747001) (end 16.207001 -13.457001) (width 0.254) (layer B.Cu) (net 9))
 (segment (start 15.08 -8.62) (end 16.207001 -9.747001) (width 0.254) (layer B.Cu) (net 9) (status 10))
 (via (at 6.5 -12.5) (size 0.6) (drill 0.4) (layers F.Cu B.Cu) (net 9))
 (segment (start 2.25 -12.5) (end 6.5 -12.5) (width 0.3048) (layer B.Cu) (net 9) (status 10))
 (segment (start 35.4 -19.12) (end 35.4 -15.65) (width 0.254) (layer B.Cu) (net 9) (status 10))
 (segment (start 35.4 -15.65) (end 34 -14.25) (width 0.254) (layer B.Cu) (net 9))
 (segment (start 17 -14.25) (end 16.5 -13.75) (width 0.254) (layer B.Cu) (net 9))
 (segment (start 34 -14.25) (end 17 -14.25) (width 0.254) (layer B.Cu) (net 9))
 (segment (start 16.207001 -13.457001) (end 16.5 -13.75) (width 0.254) (layer B.Cu) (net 9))
 (segment (start 15.08 -8.62) (end 13.75 -9.95) (width 0.254) (layer F.Cu) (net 9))
 (segment (start 13.75 -9.95) (end 13.75 -12.75) (width 0.254) (layer F.Cu) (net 9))
 (segment (start 13.75 -12.75) (end 12.75 -13.75) (width 0.254) (layer F.Cu) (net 9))
 (segment (start 9.392066 -13.75) (end 8.642066 -13) (width 0.254) (layer F.Cu) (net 9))
 (segment (start 12.75 -13.75) (end 9.392066 -13.75) (width 0.254) (layer F.Cu) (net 9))
 (segment (start 7 -13) (end 6.5 -12.5) (width 0.254) (layer F.Cu) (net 9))
 (segment (start 8.642066 -13) (end 7 -13) (width 0.254) (layer F.Cu) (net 9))
 (segment (start 35.4 -16.85) (end 35.4 -19.12) (width 0.254) (layer F.Cu) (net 9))
 (segment (start 36.75 -8.79) (end 36.75 -15.5) (width 0.254) (layer F.Cu) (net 9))
 (segment (start 38.5 -7.04) (end 36.75 -8.79) (width 0.254) (layer F.Cu) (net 9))
 (segment (start 36.75 -15.5) (end 35.4 -16.85) (width 0.254) (layer F.Cu) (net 9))
 (segment (start 40.5 -7.04) (end 38.5 -7.04) (width 0.254) (layer F.Cu) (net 9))
 (segment (start 12.54 -8.62) (end 13.75 -9.83) (width 0.254) (layer B.Cu) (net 7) (status 10))
 (segment (start 13.75 -9.83) (end 13.75 -13) (width 0.254) (layer B.Cu) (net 7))
 (segment (start 32.86 -19.12) (end 32.86 -15.81401) (width 0.254) (layer B.Cu) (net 7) (status 10))
 (segment (start 15.45401 -14.70401) (end 14.75 -14) (width 0.254) (layer B.Cu) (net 7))
 (segment (start 31.75 -14.70401) (end 15.45401 -14.70401) (width 0.254) (layer B.Cu) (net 7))
 (segment (start 32.86 -15.81401) (end 31.75 -14.70401) (width 0.254) (layer B.Cu) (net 7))
 (segment (start 13.75 -13) (end 14.75 -14) (width 0.254) (layer B.Cu) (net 7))
 (segment (start 14.85 -14.1) (end 14.875 -14.125) (width 0.254) (layer B.Cu) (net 7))
 (segment (start 10.15 -14.1) (end 14.85 -14.1) (width 0.254) (layer B.Cu) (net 7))
 (segment (start 14.75 -14) (end 14.875 -14.125) (width 0.254) (layer B.Cu) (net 7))
 (segment (start 2.25 -14.1) (end 10.15 -14.1) (width 0.254) (layer B.Cu) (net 7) (status 10))
 (segment (start 10.15 -14.1) (end 10.35 -14.1) (width 0.254) (layer B.Cu) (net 7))
 (segment (start 32.86 -19.12) (end 32.86 -16.89) (width 0.254) (layer F.Cu) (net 7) (status 10))
 (segment (start 32.86 -16.89) (end 34.25 -15.5) (width 0.254) (layer F.Cu) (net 7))
 (segment (start 34.25 -15.5) (end 34.25 -8.25) (width 0.254) (layer F.Cu) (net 7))
 (segment (start 34.25 -8.25) (end 38 -4.5) (width 0.254) (layer F.Cu) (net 7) (status 20))
 (segment (start 40.5 -4.5) (end 38.25 -4.5) (width 0.254) (layer F.Cu) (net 7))
 (segment (start 38.25 -4.5) (end 38.5 -4.5) (width 0.254) (layer F.Cu) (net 7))
 (segment (start 38 -4.5) (end 38.25 -4.5) (width 0.254) (layer F.Cu) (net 7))
 (segment (start 15.41 -5.75) (end 12.54 -8.62) (width 0.254) (layer F.Cu) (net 7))
 (segment (start 22 -5) (end 21.25 -5.75) (width 0.254) (layer F.Cu) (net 7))
 (segment (start 21.25 -5.75) (end 15.41 -5.75) (width 0.254) (layer F.Cu) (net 7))
 (segment (start 22 -3) (end 22 -5) (width 0.254) (layer F.Cu) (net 7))
 (segment (start 22.75 -2.25) (end 22 -3) (width 0.254) (layer F.Cu) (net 7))
 (segment (start 22.75 -2) (end 22.75 -2.25) (width 0.254) (layer F.Cu) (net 7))
 (segment (start 17.62 -8.62) (end 18.12 -8.62) (width 0.254) (layer B.Cu) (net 8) (status 30))
 (segment (start 18.12 -8.62) (end 19 -9.5) (width 0.254) (layer B.Cu) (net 8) (status 10))
 (segment (start 17.62 -7.62) (end 17.62 -8.62) (width 0.254) (layer B.Cu) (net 8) (status 20))
 (segment (start 16.75 -6.75) (end 17.62 -7.62) (width 0.254) (layer B.Cu) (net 8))
 (segment (start 12 -6.75) (end 16.75 -6.75) (width 0.254) (layer B.Cu) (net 8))
 (segment (start 11.412999 -7.337001) (end 12 -6.75) (width 0.254) (layer B.Cu) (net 8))
 (segment (start 11.412999 -12.337001) (end 11.412999 -7.337001) (width 0.254) (layer B.Cu) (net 8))
 (segment (start 10.45 -13.3) (end 11.412999 -12.337001) (width 0.254) (layer B.Cu) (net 8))
 (segment (start 2.25 -13.3) (end 10.45 -13.3) (width 0.254) (layer B.Cu) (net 8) (status 10))
 (segment (start 20 -13.75) (end 19 -12.75) (width 0.254) (layer B.Cu) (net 8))
 (segment (start 35.75 -13.75) (end 20 -13.75) (width 0.254) (layer B.Cu) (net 8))
 (segment (start 37.94 -15.94) (end 35.75 -13.75) (width 0.254) (layer B.Cu) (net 8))
 (segment (start 37.94 -19.12) (end 37.94 -15.94) (width 0.254) (layer B.Cu) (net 8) (status 10))
 (segment (start 19 -9.5) (end 19 -12.75) (width 0.254) (layer B.Cu) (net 8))
 (segment (start 43.04 -4.5) (end 45 -6.46) (width 0.254) (layer F.Cu) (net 8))
 (segment (start 45 -12.06) (end 37.94 -19.12) (width 0.254) (layer F.Cu) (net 8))
 (segment (start 45 -6.46) (end 45 -12.06) (width 0.254) (layer F.Cu) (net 8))
 (segment (start 2.25 -3.7) (end 8.05 -3.7) (width 0.254) (layer B.Cu) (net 12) (status 10))
 (segment (start 10 -1.75) (end 10 -1) (width 0.254) (layer B.Cu) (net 12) (status 30))
 (segment (start 8.05 -3.7) (end 10 -1.75) (width 0.254) (layer B.Cu) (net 12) (status 20))
 (segment (start 39.29481 -0.75481) (end 40.5 -1.96) (width 0.254) (layer B.Cu) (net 12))
 (segment (start 20.74519 -0.75481) (end 39.29481 -0.75481) (width 0.254) (layer B.Cu) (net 12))
 (segment (start 10 -1) (end 11.5 -2.5) (width 0.254) (layer B.Cu) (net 12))
 (segment (start 20.70401 -0.80561) (end 20.99519 -0.80561) (width 0.3556) (layer B.Cu) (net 12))
 (segment (start 20.55561 -0.80561) (end 18.86122 -2.5) (width 0.254) (layer B.Cu) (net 12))
 (segment (start 20.70401 -0.80561) (end 20.55561 -0.80561) (width 0.254) (layer B.Cu) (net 12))
 (segment (start 18.86122 -2.5) (end 18.75 -2.5) (width 0.254) (layer B.Cu) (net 12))
 (segment (start 18.75 -2.5) (end 19 -2.5) (width 0.254) (layer B.Cu) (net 12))
 (segment (start 11.5 -2.5) (end 18.75 -2.5) (width 0.254) (layer B.Cu) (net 12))
 (segment (start 10 -11.5) (end 9.75 -11.5) (width 0.254) (layer B.Cu) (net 12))
 (segment (start 9.75 -11.5) (end 8.25 -10) (width 0.254) (layer B.Cu) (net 12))
 (via (at 10 -5) (size 0.6) (drill 0.4) (layers F.Cu B.Cu) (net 12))
 (segment (start 8.25 -6.75) (end 10 -5) (width 0.254) (layer B.Cu) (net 12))
 (segment (start 8.25 -10) (end 8.25 -6.75) (width 0.254) (layer B.Cu) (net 12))
 (segment (start 10 -5) (end 10 -1) (width 0.254) (layer F.Cu) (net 12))
 (segment (start 28.8 -9.98) (end 30.32 -11.5) (width 0.254) (layer F.Cu) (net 16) (status 20))
 (segment (start 28.8 -9) (end 28.8 -9.98) (width 0.254) (layer F.Cu) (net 16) (status 10))
 (segment (start 31.2 -9.84) (end 32.86 -11.5) (width 0.254) (layer F.Cu) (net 17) (status 30))
 (segment (start 31.2 -9) (end 31.2 -9.84) (width 0.254) (layer F.Cu) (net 17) (status 30))
 (segment (start 21.25 -2) (end 21.25 -4) (width 0.254) (layer F.Cu) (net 14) (status 30))
 (segment (start 2.25 -16.5) (end 6.5 -16.5) (width 0.3556) (layer B.Cu) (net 5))
 (via (at 7.5 -18) (size 0.6) (drill 0.4) (layers F.Cu B.Cu) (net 5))
 (segment (start 7.5 -17.5) (end 7.5 -18) (width 0.3556) (layer B.Cu) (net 5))
 (segment (start 6.5 -16.5) (end 7.5 -17.5) (width 0.3556) (layer B.Cu) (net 5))
 (segment (start 7.5 -18) (end 7.5 -16.625) (width 0.3556) (layer F.Cu) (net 5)))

